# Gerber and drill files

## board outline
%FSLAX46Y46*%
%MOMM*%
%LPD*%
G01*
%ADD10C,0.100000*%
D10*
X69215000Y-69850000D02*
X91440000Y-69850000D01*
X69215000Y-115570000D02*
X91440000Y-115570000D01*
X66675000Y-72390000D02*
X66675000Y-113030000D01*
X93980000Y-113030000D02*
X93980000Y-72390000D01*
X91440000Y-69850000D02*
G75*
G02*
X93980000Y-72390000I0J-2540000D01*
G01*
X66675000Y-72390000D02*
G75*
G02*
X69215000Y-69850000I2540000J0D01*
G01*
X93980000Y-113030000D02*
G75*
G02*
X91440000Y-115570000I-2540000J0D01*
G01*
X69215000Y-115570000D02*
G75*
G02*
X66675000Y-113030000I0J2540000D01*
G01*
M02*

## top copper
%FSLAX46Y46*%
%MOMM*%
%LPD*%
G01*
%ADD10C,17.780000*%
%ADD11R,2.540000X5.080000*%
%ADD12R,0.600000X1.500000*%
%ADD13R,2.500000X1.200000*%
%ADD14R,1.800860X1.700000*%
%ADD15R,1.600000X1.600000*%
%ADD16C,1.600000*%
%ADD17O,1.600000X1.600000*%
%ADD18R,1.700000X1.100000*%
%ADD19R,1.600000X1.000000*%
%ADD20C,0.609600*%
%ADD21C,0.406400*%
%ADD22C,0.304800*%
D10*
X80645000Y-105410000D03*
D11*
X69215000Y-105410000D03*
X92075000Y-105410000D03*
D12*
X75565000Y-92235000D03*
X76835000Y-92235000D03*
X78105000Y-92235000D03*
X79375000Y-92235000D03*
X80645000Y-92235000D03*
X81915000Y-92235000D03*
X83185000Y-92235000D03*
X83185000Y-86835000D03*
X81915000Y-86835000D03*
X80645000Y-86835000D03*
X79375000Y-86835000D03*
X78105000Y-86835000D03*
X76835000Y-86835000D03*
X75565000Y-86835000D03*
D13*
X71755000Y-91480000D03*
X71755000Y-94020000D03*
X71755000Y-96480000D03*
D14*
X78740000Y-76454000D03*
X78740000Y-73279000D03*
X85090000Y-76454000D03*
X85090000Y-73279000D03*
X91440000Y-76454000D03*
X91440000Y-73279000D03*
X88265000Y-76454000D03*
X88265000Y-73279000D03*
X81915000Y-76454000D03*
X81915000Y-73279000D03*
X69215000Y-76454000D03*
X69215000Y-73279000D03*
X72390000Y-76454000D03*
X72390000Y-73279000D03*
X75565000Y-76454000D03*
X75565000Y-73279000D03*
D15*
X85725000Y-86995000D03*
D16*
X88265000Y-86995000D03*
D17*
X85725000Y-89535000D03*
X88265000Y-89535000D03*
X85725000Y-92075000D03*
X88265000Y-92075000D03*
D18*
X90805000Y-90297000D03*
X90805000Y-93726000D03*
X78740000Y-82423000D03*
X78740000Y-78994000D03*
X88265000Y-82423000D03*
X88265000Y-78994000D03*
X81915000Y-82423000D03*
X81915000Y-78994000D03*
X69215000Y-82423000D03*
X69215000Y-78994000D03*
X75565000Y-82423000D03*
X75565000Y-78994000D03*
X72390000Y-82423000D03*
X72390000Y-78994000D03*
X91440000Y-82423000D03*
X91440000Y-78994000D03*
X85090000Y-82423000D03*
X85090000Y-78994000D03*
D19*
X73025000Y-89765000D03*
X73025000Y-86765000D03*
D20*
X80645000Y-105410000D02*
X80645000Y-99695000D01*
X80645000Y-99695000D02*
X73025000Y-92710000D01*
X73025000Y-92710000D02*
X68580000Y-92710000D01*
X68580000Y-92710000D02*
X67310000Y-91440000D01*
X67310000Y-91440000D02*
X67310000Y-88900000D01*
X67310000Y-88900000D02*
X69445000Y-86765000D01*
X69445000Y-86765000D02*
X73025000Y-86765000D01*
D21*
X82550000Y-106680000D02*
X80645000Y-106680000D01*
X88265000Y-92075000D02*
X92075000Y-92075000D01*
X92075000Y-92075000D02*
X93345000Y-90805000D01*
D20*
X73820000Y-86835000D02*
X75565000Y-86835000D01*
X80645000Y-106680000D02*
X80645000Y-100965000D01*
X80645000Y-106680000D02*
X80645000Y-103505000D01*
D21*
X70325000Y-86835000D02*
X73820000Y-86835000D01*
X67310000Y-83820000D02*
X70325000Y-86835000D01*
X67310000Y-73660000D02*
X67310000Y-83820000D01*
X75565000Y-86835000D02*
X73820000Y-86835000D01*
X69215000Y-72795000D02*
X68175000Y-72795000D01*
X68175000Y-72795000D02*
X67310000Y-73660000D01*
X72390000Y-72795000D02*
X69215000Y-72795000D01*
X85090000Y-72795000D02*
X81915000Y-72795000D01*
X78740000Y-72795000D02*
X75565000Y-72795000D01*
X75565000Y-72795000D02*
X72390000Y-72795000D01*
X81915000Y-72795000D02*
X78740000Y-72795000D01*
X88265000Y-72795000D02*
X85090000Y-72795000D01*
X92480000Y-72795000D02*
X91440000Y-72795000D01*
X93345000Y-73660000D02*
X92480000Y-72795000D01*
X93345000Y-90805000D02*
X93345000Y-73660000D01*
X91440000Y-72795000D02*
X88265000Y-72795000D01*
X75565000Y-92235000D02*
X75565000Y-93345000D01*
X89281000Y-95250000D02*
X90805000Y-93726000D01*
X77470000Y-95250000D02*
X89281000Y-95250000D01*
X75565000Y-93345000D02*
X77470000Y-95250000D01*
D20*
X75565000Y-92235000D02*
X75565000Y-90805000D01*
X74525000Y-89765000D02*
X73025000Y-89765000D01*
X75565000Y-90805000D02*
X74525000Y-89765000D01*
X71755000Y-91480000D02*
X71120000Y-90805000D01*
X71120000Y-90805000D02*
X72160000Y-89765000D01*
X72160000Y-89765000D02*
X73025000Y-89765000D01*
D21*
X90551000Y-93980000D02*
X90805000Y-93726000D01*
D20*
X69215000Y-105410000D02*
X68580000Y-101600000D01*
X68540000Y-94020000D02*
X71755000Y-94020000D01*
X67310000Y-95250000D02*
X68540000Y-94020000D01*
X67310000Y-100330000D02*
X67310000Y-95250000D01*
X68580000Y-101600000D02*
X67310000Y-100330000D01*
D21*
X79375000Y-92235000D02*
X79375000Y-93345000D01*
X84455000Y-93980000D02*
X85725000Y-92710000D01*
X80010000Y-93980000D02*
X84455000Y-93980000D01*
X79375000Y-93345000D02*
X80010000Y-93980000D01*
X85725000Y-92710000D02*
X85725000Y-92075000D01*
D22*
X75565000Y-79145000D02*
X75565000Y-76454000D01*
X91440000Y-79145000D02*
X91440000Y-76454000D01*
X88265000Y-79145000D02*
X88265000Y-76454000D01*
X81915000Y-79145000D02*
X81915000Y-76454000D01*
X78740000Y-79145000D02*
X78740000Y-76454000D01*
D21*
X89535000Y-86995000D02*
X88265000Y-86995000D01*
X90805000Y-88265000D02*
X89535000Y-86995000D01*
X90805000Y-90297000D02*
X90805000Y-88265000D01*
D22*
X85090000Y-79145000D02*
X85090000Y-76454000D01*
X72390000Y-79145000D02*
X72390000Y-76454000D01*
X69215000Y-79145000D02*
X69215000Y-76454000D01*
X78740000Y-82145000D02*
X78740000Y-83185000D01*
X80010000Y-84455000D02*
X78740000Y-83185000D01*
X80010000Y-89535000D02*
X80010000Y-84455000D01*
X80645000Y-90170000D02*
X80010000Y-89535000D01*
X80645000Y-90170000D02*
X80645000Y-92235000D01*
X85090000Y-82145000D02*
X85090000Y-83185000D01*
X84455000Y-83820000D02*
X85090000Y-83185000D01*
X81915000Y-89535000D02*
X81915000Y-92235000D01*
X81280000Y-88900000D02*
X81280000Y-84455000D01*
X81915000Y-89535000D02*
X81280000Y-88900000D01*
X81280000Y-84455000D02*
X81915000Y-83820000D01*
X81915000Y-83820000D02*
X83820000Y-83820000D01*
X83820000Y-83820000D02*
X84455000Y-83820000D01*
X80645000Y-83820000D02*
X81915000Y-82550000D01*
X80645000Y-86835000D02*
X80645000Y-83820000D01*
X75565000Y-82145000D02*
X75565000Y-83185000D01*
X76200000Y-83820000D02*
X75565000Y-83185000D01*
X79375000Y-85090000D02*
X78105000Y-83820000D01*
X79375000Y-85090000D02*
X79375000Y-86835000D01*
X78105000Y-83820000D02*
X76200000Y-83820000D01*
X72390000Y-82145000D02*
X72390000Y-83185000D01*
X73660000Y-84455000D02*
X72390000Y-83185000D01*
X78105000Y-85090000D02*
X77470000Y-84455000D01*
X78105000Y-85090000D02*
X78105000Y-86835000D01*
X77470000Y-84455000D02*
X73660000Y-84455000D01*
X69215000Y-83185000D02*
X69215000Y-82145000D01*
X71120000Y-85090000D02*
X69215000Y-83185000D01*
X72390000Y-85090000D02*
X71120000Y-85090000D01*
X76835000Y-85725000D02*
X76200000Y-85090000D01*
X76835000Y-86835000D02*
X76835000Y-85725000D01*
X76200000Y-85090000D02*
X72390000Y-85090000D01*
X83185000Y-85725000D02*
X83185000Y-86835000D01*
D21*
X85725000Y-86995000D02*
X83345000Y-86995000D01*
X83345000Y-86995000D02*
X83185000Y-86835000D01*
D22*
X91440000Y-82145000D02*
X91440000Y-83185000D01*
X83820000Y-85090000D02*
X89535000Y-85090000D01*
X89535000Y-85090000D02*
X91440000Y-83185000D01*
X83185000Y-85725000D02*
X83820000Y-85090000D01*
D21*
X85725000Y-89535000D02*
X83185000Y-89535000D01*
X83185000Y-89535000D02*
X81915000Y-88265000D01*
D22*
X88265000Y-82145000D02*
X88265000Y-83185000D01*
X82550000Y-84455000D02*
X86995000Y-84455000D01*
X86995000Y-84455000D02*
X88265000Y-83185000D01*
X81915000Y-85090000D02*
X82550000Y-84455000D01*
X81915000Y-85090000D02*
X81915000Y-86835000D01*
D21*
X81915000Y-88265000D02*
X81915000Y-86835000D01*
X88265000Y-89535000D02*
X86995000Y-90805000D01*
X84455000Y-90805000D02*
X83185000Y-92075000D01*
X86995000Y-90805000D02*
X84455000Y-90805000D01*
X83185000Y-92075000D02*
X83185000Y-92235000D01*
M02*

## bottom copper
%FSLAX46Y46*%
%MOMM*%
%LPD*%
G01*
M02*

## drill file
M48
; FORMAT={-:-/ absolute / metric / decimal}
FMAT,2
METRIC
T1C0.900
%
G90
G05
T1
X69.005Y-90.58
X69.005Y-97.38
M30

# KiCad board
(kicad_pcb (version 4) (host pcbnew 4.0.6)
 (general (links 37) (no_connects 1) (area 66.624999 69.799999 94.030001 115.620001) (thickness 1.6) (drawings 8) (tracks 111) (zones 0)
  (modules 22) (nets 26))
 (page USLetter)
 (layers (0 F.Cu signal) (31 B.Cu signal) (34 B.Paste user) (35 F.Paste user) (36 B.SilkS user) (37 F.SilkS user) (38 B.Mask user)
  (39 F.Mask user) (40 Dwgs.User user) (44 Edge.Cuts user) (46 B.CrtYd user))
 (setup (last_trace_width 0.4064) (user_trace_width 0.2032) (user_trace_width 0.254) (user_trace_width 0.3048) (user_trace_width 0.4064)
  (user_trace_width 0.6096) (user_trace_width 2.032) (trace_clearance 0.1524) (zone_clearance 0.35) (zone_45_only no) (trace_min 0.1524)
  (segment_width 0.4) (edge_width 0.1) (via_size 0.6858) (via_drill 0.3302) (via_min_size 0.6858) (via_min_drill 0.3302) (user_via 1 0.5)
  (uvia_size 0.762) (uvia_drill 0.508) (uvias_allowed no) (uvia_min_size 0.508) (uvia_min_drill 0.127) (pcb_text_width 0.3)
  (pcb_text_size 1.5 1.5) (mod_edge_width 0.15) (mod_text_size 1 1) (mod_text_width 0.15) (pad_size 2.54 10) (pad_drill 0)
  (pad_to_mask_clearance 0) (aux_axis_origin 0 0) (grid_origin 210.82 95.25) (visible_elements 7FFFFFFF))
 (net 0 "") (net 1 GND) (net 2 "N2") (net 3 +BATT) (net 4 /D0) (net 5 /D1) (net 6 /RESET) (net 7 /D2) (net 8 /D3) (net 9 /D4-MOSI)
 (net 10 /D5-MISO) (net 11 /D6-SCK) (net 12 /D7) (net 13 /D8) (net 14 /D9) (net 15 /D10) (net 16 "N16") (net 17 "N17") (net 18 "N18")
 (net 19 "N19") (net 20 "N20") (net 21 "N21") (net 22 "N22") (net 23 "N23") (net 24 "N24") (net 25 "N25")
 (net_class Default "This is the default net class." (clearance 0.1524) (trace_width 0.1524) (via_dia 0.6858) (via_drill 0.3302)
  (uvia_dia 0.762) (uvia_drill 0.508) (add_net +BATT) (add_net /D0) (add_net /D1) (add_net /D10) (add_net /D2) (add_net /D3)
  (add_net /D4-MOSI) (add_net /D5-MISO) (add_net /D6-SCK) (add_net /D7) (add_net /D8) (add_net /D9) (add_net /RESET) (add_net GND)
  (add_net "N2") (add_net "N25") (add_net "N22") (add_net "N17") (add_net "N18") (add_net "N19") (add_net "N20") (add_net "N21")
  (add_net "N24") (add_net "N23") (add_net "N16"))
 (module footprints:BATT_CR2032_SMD (layer F.Cu) (at 80.645 105.41)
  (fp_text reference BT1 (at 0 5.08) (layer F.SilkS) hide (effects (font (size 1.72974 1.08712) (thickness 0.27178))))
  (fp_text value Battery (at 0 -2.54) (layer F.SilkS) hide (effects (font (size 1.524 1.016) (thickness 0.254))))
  (pad 2 smd circle (at 0 0) (size 17.78 17.78) (layers F.Cu F.Paste F.Mask) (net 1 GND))
  (pad 1 smd rect (at -11.43 0) (size 2.54 5.08) (layers F.Cu F.Paste F.Mask) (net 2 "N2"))
  (pad 1 smd rect (at 11.43 0) (size 2.54 5.08) (layers F.Cu F.Paste F.Mask) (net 2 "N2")))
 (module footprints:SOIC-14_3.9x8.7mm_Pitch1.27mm (layer F.Cu) (at 79.375 89.535 90)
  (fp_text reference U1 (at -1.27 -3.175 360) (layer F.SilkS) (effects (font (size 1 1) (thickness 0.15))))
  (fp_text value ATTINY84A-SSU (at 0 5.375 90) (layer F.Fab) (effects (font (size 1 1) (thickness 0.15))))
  (pad 1 smd rect (at -2.7 -3.81 90) (size 1.5 0.6) (layers F.Cu F.Paste F.Mask) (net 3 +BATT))
  (pad 2 smd rect (at -2.7 -2.54 90) (size 1.5 0.6) (layers F.Cu F.Paste F.Mask) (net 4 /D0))
  (pad 3 smd rect (at -2.7 -1.27 90) (size 1.5 0.6) (layers F.Cu F.Paste F.Mask) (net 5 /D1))
  (pad 4 smd rect (at -2.7 0 90) (size 1.5 0.6) (layers F.Cu F.Paste F.Mask) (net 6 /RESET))
  (pad 5 smd rect (at -2.7 1.27 90) (size 1.5 0.6) (layers F.Cu F.Paste F.Mask) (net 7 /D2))
  (pad 6 smd rect (at -2.7 2.54 90) (size 1.5 0.6) (layers F.Cu F.Paste F.Mask) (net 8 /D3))
  (pad 7 smd rect (at -2.7 3.81 90) (size 1.5 0.6) (layers F.Cu F.Paste F.Mask) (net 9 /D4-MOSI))
  (pad 8 smd rect (at 2.7 3.81 90) (size 1.5 0.6) (layers F.Cu F.Paste F.Mask) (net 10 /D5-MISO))
  (pad 9 smd rect (at 2.7 2.54 90) (size 1.5 0.6) (layers F.Cu F.Paste F.Mask) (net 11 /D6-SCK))
  (pad 10 smd rect (at 2.7 1.27 90) (size 1.5 0.6) (layers F.Cu F.Paste F.Mask) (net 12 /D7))
  (pad 11 smd rect (at 2.7 0 90) (size 1.5 0.6) (layers F.Cu F.Paste F.Mask) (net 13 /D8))
  (pad 12 smd rect (at 2.7 -1.27 90) (size 1.5 0.6) (layers F.Cu F.Paste F.Mask) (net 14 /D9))
  (pad 13 smd rect (at 2.7 -2.54 90) (size 1.5 0.6) (layers F.Cu F.Paste F.Mask) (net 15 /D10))
  (pad 14 smd rect (at 2.7 -3.81 90) (size 1.5 0.6) (layers F.Cu F.Paste F.Mask) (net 1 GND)))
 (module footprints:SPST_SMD (layer F.Cu) (at 71.755 93.98 270)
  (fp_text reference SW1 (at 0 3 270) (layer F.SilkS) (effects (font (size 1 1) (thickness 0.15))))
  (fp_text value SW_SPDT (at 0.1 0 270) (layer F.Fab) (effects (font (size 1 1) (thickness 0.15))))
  (pad "" np_thru_hole circle (at 3.4 2.75 270) (size 0.9 0.9) (drill 0.9) (layers *.Cu *.Mask))
  (pad 3 smd rect (at -2.5 0 270) (size 1.2 2.5) (layers F.Cu F.Paste F.Mask) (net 3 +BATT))
  (pad 1 smd rect (at 0.04 0 270) (size 1.2 2.5) (layers F.Cu F.Paste F.Mask) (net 2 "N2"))
  (pad 2 smd rect (at 2.5 0 270) (size 1.2 2.5) (layers F.Cu F.Paste F.Mask) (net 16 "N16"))
  (pad "" np_thru_hole circle (at -3.4 2.75 270) (size 0.9 0.9) (drill 0.9) (layers *.Cu *.Mask)))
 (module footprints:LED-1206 (layer F.Cu) (at 78.74 74.93 270)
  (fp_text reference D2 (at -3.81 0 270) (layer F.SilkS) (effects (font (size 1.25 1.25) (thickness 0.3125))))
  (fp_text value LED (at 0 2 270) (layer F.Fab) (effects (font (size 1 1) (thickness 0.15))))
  (pad 2 smd rect (at 1.524 0 90) (size 1.7 1.80086) (layers F.Cu F.Paste F.Mask) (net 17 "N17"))
  (pad 1 smd rect (at -1.651 0 90) (size 1.7 1.80086) (layers F.Cu F.Paste F.Mask) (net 1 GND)))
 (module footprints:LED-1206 (layer F.Cu) (at 85.09 74.93 270)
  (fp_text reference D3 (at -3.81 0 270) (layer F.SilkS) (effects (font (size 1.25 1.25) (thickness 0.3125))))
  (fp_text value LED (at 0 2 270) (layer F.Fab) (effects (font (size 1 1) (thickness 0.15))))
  (pad 2 smd rect (at 1.524 0 90) (size 1.7 1.80086) (layers F.Cu F.Paste F.Mask) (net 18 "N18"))
  (pad 1 smd rect (at -1.651 0 90) (size 1.7 1.80086) (layers F.Cu F.Paste F.Mask) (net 1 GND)))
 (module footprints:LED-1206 (layer F.Cu) (at 91.44 74.93 270)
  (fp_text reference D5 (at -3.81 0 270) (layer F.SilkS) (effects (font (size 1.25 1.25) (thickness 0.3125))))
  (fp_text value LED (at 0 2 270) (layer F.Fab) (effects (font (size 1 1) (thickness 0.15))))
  (pad 2 smd rect (at 1.524 0 90) (size 1.7 1.80086) (layers F.Cu F.Paste F.Mask) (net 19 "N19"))
  (pad 1 smd rect (at -1.651 0 90) (size 1.7 1.80086) (layers F.Cu F.Paste F.Mask) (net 1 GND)))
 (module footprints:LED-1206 (layer F.Cu) (at 88.265 74.93 270)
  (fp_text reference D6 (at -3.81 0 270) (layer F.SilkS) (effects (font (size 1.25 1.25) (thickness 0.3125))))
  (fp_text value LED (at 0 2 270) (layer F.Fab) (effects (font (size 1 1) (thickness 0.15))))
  (pad 2 smd rect (at 1.524 0 90) (size 1.7 1.80086) (layers F.Cu F.Paste F.Mask) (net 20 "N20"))
  (pad 1 smd rect (at -1.651 0 90) (size 1.7 1.80086) (layers F.Cu F.Paste F.Mask) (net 1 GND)))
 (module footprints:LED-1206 (layer F.Cu) (at 81.915 74.93 270)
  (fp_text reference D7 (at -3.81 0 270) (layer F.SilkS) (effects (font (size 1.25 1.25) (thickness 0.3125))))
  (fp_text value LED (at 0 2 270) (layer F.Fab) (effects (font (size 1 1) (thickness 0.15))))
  (pad 2 smd rect (at 1.524 0 90) (size 1.7 1.80086) (layers F.Cu F.Paste F.Mask) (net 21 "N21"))
  (pad 1 smd rect (at -1.651 0 90) (size 1.7 1.80086) (layers F.Cu F.Paste F.Mask) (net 1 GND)))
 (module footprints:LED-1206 (layer F.Cu) (at 69.215 74.93 270)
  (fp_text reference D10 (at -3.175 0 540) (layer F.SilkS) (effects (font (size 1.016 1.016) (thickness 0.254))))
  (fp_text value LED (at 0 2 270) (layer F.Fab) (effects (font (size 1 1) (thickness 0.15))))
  (pad 2 smd rect (at 1.524 0 90) (size 1.7 1.80086) (layers F.Cu F.Paste F.Mask) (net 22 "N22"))
  (pad 1 smd rect (at -1.651 0 90) (size 1.7 1.80086) (layers F.Cu F.Paste F.Mask) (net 1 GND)))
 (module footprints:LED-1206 (layer F.Cu) (at 72.39 74.93 270)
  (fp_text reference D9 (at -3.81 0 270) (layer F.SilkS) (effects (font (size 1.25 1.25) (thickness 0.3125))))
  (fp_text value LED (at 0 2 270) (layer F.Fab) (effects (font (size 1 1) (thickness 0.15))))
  (pad 2 smd rect (at 1.524 0 90) (size 1.7 1.80086) (layers F.Cu F.Paste F.Mask) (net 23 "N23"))
  (pad 1 smd rect (at -1.651 0 90) (size 1.7 1.80086) (layers F.Cu F.Paste F.Mask) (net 1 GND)))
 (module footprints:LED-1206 (layer F.Cu) (at 75.565 74.93 270)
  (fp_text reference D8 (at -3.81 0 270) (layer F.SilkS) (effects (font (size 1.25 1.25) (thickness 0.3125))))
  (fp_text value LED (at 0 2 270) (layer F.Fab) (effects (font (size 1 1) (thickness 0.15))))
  (pad 2 smd rect (at 1.524 0 90) (size 1.7 1.80086) (layers F.Cu F.Paste F.Mask) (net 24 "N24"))
  (pad 1 smd rect (at -1.651 0 90) (size 1.7 1.80086) (layers F.Cu F.Paste F.Mask) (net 1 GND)))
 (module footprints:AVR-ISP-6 (layer F.Cu) (at 85.725 86.995)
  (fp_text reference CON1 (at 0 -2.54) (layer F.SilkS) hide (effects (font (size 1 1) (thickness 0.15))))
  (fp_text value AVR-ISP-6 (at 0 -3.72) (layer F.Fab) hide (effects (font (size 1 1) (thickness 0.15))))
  (pad 1 smd rect (at 0 0) (size 1.6 1.6) (layers F.Cu F.Paste F.Mask) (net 10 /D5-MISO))
  (pad 2 smd circle (at 2.54 0) (size 1.6 1.6) (layers F.Cu F.Paste F.Mask) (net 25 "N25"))
  (pad 3 smd oval (at 0 2.54) (size 1.6 1.6) (layers F.Cu F.Paste F.Mask) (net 11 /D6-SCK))
  (pad 4 smd oval (at 2.54 2.54) (size 1.6 1.6) (layers F.Cu F.Paste F.Mask) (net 9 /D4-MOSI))
  (pad 5 smd oval (at 0 5.08) (size 1.6 1.6) (layers F.Cu F.Paste F.Mask) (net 6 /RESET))
  (pad 6 smd oval (at 2.54 5.08) (size 1.6 1.6) (layers F.Cu F.Paste F.Mask) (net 1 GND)))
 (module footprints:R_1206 (layer F.Cu) (at 90.805 92.075 270)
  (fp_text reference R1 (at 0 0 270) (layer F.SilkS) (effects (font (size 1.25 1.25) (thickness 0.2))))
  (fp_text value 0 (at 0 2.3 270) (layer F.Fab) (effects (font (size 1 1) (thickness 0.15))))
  (pad 1 smd rect (at -1.778 0 270) (size 1.1 1.7) (layers F.Cu F.Paste F.Mask) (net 25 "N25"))
  (pad 2 smd rect (at 1.651 0 270) (size 1.1 1.7) (layers F.Cu F.Paste F.Mask) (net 3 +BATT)))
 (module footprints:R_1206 (layer F.Cu) (at 78.74 80.645 90)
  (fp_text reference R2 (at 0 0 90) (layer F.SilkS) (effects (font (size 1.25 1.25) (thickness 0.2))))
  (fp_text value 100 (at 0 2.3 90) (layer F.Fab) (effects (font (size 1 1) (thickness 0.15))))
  (pad 1 smd rect (at -1.778 0 90) (size 1.1 1.7) (layers F.Cu F.Paste F.Mask) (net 7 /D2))
  (pad 2 smd rect (at 1.651 0 90) (size 1.1 1.7) (layers F.Cu F.Paste F.Mask) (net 17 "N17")))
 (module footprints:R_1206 (layer F.Cu) (at 88.265 80.645 90)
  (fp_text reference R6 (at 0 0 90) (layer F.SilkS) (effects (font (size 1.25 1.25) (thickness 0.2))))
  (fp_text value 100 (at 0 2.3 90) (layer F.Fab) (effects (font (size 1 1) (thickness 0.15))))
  (pad 1 smd rect (at -1.778 0 90) (size 1.1 1.7) (layers F.Cu F.Paste F.Mask) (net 11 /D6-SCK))
  (pad 2 smd rect (at 1.651 0 90) (size 1.1 1.7) (layers F.Cu F.Paste F.Mask) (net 20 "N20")))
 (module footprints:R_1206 (layer F.Cu) (at 81.915 80.645 90)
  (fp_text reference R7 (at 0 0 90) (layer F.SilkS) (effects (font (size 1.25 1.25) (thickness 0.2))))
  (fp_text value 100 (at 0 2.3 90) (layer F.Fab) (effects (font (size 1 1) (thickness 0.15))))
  (pad 1 smd rect (at -1.778 0 90) (size 1.1 1.7) (layers F.Cu F.Paste F.Mask) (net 12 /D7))
  (pad 2 smd rect (at 1.651 0 90) (size 1.1 1.7) (layers F.Cu F.Paste F.Mask) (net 21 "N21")))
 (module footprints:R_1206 (layer F.Cu) (at 69.215 80.645 90)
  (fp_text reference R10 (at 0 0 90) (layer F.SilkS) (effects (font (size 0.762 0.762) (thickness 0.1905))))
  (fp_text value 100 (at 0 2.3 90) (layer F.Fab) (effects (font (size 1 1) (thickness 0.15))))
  (pad 1 smd rect (at -1.778 0 90) (size 1.1 1.7) (layers F.Cu F.Paste F.Mask) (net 15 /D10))
  (pad 2 smd rect (at 1.651 0 90) (size 1.1 1.7) (layers F.Cu F.Paste F.Mask) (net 22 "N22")))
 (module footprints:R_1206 (layer F.Cu) (at 75.565 80.645 90)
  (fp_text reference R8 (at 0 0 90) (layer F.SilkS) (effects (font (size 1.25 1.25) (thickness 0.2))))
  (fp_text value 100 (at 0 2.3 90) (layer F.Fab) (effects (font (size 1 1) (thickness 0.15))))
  (pad 1 smd rect (at -1.778 0 90) (size 1.1 1.7) (layers F.Cu F.Paste F.Mask) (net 13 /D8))
  (pad 2 smd rect (at 1.651 0 90) (size 1.1 1.7) (layers F.Cu F.Paste F.Mask) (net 24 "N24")))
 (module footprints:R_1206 (layer F.Cu) (at 72.39 80.645 90)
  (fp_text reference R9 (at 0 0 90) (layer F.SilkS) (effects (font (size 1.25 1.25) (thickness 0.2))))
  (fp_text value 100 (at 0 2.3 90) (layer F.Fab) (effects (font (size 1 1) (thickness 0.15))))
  (pad 1 smd rect (at -1.778 0 90) (size 1.1 1.7) (layers F.Cu F.Paste F.Mask) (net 14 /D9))
  (pad 2 smd rect (at 1.651 0 90) (size 1.1 1.7) (layers F.Cu F.Paste F.Mask) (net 23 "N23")))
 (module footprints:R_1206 (layer F.Cu) (at 91.44 80.645 90)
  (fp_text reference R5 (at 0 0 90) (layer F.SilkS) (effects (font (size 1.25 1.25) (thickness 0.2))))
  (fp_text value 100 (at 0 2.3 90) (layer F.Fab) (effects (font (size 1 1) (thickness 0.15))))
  (pad 1 smd rect (at -1.778 0 90) (size 1.1 1.7) (layers F.Cu F.Paste F.Mask) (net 10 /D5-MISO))
  (pad 2 smd rect (at 1.651 0 90) (size 1.1 1.7) (layers F.Cu F.Paste F.Mask) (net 19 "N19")))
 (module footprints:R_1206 (layer F.Cu) (at 85.09 80.645 90)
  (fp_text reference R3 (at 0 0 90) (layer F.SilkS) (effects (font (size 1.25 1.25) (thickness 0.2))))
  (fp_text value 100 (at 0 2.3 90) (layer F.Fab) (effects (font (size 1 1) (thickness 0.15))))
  (pad 1 smd rect (at -1.778 0 90) (size 1.1 1.7) (layers F.Cu F.Paste F.Mask) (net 8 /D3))
  (pad 2 smd rect (at 1.651 0 90) (size 1.1 1.7) (layers F.Cu F.Paste F.Mask) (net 18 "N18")))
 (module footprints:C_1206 (layer F.Cu) (at 73.025 88.265 90)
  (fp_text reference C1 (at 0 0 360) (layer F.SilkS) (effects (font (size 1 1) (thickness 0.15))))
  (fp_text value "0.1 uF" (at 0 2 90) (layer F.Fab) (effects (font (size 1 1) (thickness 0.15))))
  (pad 1 smd rect (at -1.5 0 90) (size 1 1.6) (layers F.Cu F.Paste F.Mask) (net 3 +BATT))
  (pad 2 smd rect (at 1.5 0 90) (size 1 1.6) (layers F.Cu F.Paste F.Mask) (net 1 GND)))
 (gr_line (start 69.215 69.85) (end 91.44 69.85) (angle 90) (layer Edge.Cuts) (width 0.1))
 (gr_line (start 69.215 115.57) (end 91.44 115.57) (angle 90) (layer Edge.Cuts) (width 0.1))
 (gr_line (start 66.675 72.39) (end 66.675 113.03) (angle 90) (layer Edge.Cuts) (width 0.1))
 (gr_line (start 93.98 113.03) (end 93.98 72.39) (angle 90) (layer Edge.Cuts) (width 0.1))
 (gr_arc (start 91.44 72.39) (end 91.44 69.85) (angle 90) (layer Edge.Cuts) (width 0.1))
 (gr_arc (start 69.215 72.39) (end 66.675 72.39) (angle 90) (layer Edge.Cuts) (width 0.1))
 (gr_arc (start 91.44 113.03) (end 93.98 113.03) (angle 90) (layer Edge.Cuts) (width 0.1))
 (gr_arc (start 69.215 113.03) (end 69.215 115.57) (angle 90) (layer Edge.Cuts) (width 0.1))
 (segment (start 80.645 105.41) (end 80.645 99.695) (width 0.6096) (layer F.Cu) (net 1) (status 30))
 (segment (start 80.645 99.695) (end 73.025 92.71) (width 0.6096) (layer F.Cu) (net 1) (status 10))
 (segment (start 73.025 92.71) (end 68.58 92.71) (width 0.6096) (layer F.Cu) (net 1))
 (segment (start 68.58 92.71) (end 67.31 91.44) (width 0.6096) (layer F.Cu) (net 1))
 (segment (start 67.31 91.44) (end 67.31 88.9) (width 0.6096) (layer F.Cu) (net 1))
 (segment (start 67.31 88.9) (end 69.445 86.765) (width 0.6096) (layer F.Cu) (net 1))
 (segment (start 69.445 86.765) (end 73.025 86.765) (width 0.6096) (layer F.Cu) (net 1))
 (segment (start 82.55 106.68) (end 80.645 106.68) (width 0.4064) (layer F.Cu) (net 1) (status 30))
 (segment (start 88.265 92.075) (end 92.075 92.075) (width 0.4064) (layer F.Cu) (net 1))
 (segment (start 92.075 92.075) (end 93.345 90.805) (width 0.4064) (layer F.Cu) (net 1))
 (segment (start 73.82 86.835) (end 75.565 86.835) (width 0.6096) (layer F.Cu) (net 1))
 (segment (start 80.645 106.68) (end 80.645 100.965) (width 0.6096) (layer F.Cu) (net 1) (status 30))
 (segment (start 80.645 106.68) (end 80.645 103.505) (width 0.6096) (layer F.Cu) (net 1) (status 30))
 (segment (start 70.325 86.835) (end 73.82 86.835) (width 0.4064) (layer F.Cu) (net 1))
 (segment (start 67.31 83.82) (end 70.325 86.835) (width 0.4064) (layer F.Cu) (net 1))
 (segment (start 67.31 73.66) (end 67.31 83.82) (width 0.4064) (layer F.Cu) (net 1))
 (segment (start 75.565 86.835) (end 73.82 86.835) (width 0.4064) (layer F.Cu) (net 1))
 (segment (start 69.215 72.795) (end 68.175 72.795) (width 0.4064) (layer F.Cu) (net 1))
 (segment (start 68.175 72.795) (end 67.31 73.66) (width 0.4064) (layer F.Cu) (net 1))
 (segment (start 72.39 72.795) (end 69.215 72.795) (width 0.4064) (layer F.Cu) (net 1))
 (segment (start 85.09 72.795) (end 81.915 72.795) (width 0.4064) (layer F.Cu) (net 1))
 (segment (start 78.74 72.795) (end 75.565 72.795) (width 0.4064) (layer F.Cu) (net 1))
 (segment (start 75.565 72.795) (end 72.39 72.795) (width 0.4064) (layer F.Cu) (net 1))
 (segment (start 81.915 72.795) (end 78.74 72.795) (width 0.4064) (layer F.Cu) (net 1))
 (segment (start 88.265 72.795) (end 85.09 72.795) (width 0.4064) (layer F.Cu) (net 1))
 (segment (start 92.48 72.795) (end 91.44 72.795) (width 0.4064) (layer F.Cu) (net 1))
 (segment (start 93.345 73.66) (end 92.48 72.795) (width 0.4064) (layer F.Cu) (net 1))
 (segment (start 93.345 90.805) (end 93.345 73.66) (width 0.4064) (layer F.Cu) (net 1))
 (segment (start 91.44 72.795) (end 88.265 72.795) (width 0.4064) (layer F.Cu) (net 1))
 (segment (start 75.565 92.235) (end 75.565 93.345) (width 0.4064) (layer F.Cu) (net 3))
 (segment (start 89.281 95.25) (end 90.805 93.726) (width 0.4064) (layer F.Cu) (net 3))
 (segment (start 77.47 95.25) (end 89.281 95.25) (width 0.4064) (layer F.Cu) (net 3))
 (segment (start 75.565 93.345) (end 77.47 95.25) (width 0.4064) (layer F.Cu) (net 3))
 (segment (start 75.565 92.235) (end 75.565 90.805) (width 0.6096) (layer F.Cu) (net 3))
 (segment (start 74.525 89.765) (end 73.025 89.765) (width 0.6096) (layer F.Cu) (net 3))
 (segment (start 75.565 90.805) (end 74.525 89.765) (width 0.6096) (layer F.Cu) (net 3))
 (segment (start 71.755 91.48) (end 71.12 90.805) (width 0.6096) (layer F.Cu) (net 3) (status 10))
 (segment (start 71.12 90.805) (end 72.16 89.765) (width 0.6096) (layer F.Cu) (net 3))
 (segment (start 72.16 89.765) (end 73.025 89.765) (width 0.6096) (layer F.Cu) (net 3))
 (segment (start 90.551 93.98) (end 90.805 93.726) (width 0.4064) (layer F.Cu) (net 3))
 (segment (start 69.215 105.41) (end 68.58 101.6) (width 0.6096) (layer F.Cu) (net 2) (status 10))
 (segment (start 68.54 94.02) (end 71.755 94.02) (width 0.6096) (layer F.Cu) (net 2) (status 20))
 (segment (start 67.31 95.25) (end 68.54 94.02) (width 0.6096) (layer F.Cu) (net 2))
 (segment (start 67.31 100.33) (end 67.31 95.25) (width 0.6096) (layer F.Cu) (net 2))
 (segment (start 68.58 101.6) (end 67.31 100.33) (width 0.6096) (layer F.Cu) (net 2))
 (segment (start 79.375 92.235) (end 79.375 93.345) (width 0.4064) (layer F.Cu) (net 6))
 (segment (start 84.455 93.98) (end 85.725 92.71) (width 0.4064) (layer F.Cu) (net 6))
 (segment (start 80.01 93.98) (end 84.455 93.98) (width 0.4064) (layer F.Cu) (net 6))
 (segment (start 79.375 93.345) (end 80.01 93.98) (width 0.4064) (layer F.Cu) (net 6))
 (segment (start 85.725 92.71) (end 85.725 92.075) (width 0.4064) (layer F.Cu) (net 6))
 (segment (start 75.565 79.145) (end 75.565 76.454) (width 0.3048) (layer F.Cu) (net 24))
 (segment (start 91.44 79.145) (end 91.44 76.454) (width 0.3048) (layer F.Cu) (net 19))
 (segment (start 88.265 79.145) (end 88.265 76.454) (width 0.3048) (layer F.Cu) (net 20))
 (segment (start 81.915 79.145) (end 81.915 76.454) (width 0.3048) (layer F.Cu) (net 21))
 (segment (start 78.74 79.145) (end 78.74 76.454) (width 0.3048) (layer F.Cu) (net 17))
 (segment (start 89.535 86.995) (end 88.265 86.995) (width 0.4064) (layer F.Cu) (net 25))
 (segment (start 90.805 88.265) (end 89.535 86.995) (width 0.4064) (layer F.Cu) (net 25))
 (segment (start 90.805 90.297) (end 90.805 88.265) (width 0.4064) (layer F.Cu) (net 25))
 (segment (start 85.09 79.145) (end 85.09 76.454) (width 0.3048) (layer F.Cu) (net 18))
 (segment (start 72.39 79.145) (end 72.39 76.454) (width 0.3048) (layer F.Cu) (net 23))
 (segment (start 69.215 79.145) (end 69.215 76.454) (width 0.3048) (layer F.Cu) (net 22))
 (segment (start 78.74 82.145) (end 78.74 83.185) (width 0.3048) (layer F.Cu) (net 7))
 (segment (start 80.01 84.455) (end 78.74 83.185) (width 0.3048) (layer F.Cu) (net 7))
 (segment (start 80.01 89.535) (end 80.01 84.455) (width 0.3048) (layer F.Cu) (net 7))
 (segment (start 80.645 90.17) (end 80.01 89.535) (width 0.3048) (layer F.Cu) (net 7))
 (segment (start 80.645 90.17) (end 80.645 92.235) (width 0.3048) (layer F.Cu) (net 7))
 (segment (start 85.09 82.145) (end 85.09 83.185) (width 0.3048) (layer F.Cu) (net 8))
 (segment (start 84.455 83.82) (end 85.09 83.185) (width 0.3048) (layer F.Cu) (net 8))
 (segment (start 81.915 89.535) (end 81.915 92.235) (width 0.3048) (layer F.Cu) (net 8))
 (segment (start 81.28 88.9) (end 81.28 84.455) (width 0.3048) (layer F.Cu) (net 8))
 (segment (start 81.915 89.535) (end 81.28 88.9) (width 0.3048) (layer F.Cu) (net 8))
 (segment (start 81.28 84.455) (end 81.915 83.82) (width 0.3048) (layer F.Cu) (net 8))
 (segment (start 81.915 83.82) (end 83.82 83.82) (width 0.3048) (layer F.Cu) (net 8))
 (segment (start 83.82 83.82) (end 84.455 83.82) (width 0.3048) (layer F.Cu) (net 8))
 (segment (start 80.645 83.82) (end 81.915 82.55) (width 0.3048) (layer F.Cu) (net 12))
 (segment (start 80.645 86.835) (end 80.645 83.82) (width 0.3048) (layer F.Cu) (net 12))
 (segment (start 75.565 82.145) (end 75.565 83.185) (width 0.3048) (layer F.Cu) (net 13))
 (segment (start 76.2 83.82) (end 75.565 83.185) (width 0.3048) (layer F.Cu) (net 13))
 (segment (start 79.375 85.09) (end 78.105 83.82) (width 0.3048) (layer F.Cu) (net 13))
 (segment (start 79.375 85.09) (end 79.375 86.835) (width 0.3048) (layer F.Cu) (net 13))
 (segment (start 78.105 83.82) (end 76.2 83.82) (width 0.3048) (layer F.Cu) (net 13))
 (segment (start 72.39 82.145) (end 72.39 83.185) (width 0.3048) (layer F.Cu) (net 14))
 (segment (start 73.66 84.455) (end 72.39 83.185) (width 0.3048) (layer F.Cu) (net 14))
 (segment (start 78.105 85.09) (end 77.47 84.455) (width 0.3048) (layer F.Cu) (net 14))
 (segment (start 78.105 85.09) (end 78.105 86.835) (width 0.3048) (layer F.Cu) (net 14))
 (segment (start 77.47 84.455) (end 73.66 84.455) (width 0.3048) (layer F.Cu) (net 14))
 (segment (start 69.215 83.185) (end 69.215 82.145) (width 0.3048) (layer F.Cu) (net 15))
 (segment (start 71.12 85.09) (end 69.215 83.185) (width 0.3048) (layer F.Cu) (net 15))
 (segment (start 72.39 85.09) (end 71.12 85.09) (width 0.3048) (layer F.Cu) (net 15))
 (segment (start 76.835 85.725) (end 76.2 85.09) (width 0.3048) (layer F.Cu) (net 15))
 (segment (start 76.835 86.835) (end 76.835 85.725) (width 0.3048) (layer F.Cu) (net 15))
 (segment (start 76.2 85.09) (end 72.39 85.09) (width 0.3048) (layer F.Cu) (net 15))
 (segment (start 83.185 85.725) (end 83.185 86.835) (width 0.3048) (layer F.Cu) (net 10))
 (segment (start 85.725 86.995) (end 83.345 86.995) (width 0.4064) (layer F.Cu) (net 10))
 (segment (start 83.345 86.995) (end 83.185 86.835) (width 0.4064) (layer F.Cu) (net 10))
 (segment (start 91.44 82.145) (end 91.44 83.185) (width 0.3048) (layer F.Cu) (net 10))
 (segment (start 83.82 85.09) (end 89.535 85.09) (width 0.3048) (layer F.Cu) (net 10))
 (segment (start 89.535 85.09) (end 91.44 83.185) (width 0.3048) (layer F.Cu) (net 10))
 (segment (start 83.185 85.725) (end 83.82 85.09) (width 0.3048) (layer F.Cu) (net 10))
 (segment (start 85.725 89.535) (end 83.185 89.535) (width 0.4064) (layer F.Cu) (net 11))
 (segment (start 83.185 89.535) (end 81.915 88.265) (width 0.4064) (layer F.Cu) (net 11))
 (segment (start 88.265 82.145) (end 88.265 83.185) (width 0.3048) (layer F.Cu) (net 11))
 (segment (start 82.55 84.455) (end 86.995 84.455) (width 0.3048) (layer F.Cu) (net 11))
 (segment (start 86.995 84.455) (end 88.265 83.185) (width 0.3048) (layer F.Cu) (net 11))
 (segment (start 81.915 85.09) (end 82.55 84.455) (width 0.3048) (layer F.Cu) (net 11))
 (segment (start 81.915 85.09) (end 81.915 86.835) (width 0.3048) (layer F.Cu) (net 11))
 (segment (start 81.915 88.265) (end 81.915 86.835) (width 0.4064) (layer F.Cu) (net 11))
 (segment (start 88.265 89.535) (end 86.995 90.805) (width 0.4064) (layer F.Cu) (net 9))
 (segment (start 84.455 90.805) (end 83.185 92.075) (width 0.4064) (layer F.Cu) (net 9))
 (segment (start 86.995 90.805) (end 84.455 90.805) (width 0.4064) (layer F.Cu) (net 9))
 (segment (start 83.185 92.075) (end 83.185 92.235) (width 0.4064) (layer F.Cu) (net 9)))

